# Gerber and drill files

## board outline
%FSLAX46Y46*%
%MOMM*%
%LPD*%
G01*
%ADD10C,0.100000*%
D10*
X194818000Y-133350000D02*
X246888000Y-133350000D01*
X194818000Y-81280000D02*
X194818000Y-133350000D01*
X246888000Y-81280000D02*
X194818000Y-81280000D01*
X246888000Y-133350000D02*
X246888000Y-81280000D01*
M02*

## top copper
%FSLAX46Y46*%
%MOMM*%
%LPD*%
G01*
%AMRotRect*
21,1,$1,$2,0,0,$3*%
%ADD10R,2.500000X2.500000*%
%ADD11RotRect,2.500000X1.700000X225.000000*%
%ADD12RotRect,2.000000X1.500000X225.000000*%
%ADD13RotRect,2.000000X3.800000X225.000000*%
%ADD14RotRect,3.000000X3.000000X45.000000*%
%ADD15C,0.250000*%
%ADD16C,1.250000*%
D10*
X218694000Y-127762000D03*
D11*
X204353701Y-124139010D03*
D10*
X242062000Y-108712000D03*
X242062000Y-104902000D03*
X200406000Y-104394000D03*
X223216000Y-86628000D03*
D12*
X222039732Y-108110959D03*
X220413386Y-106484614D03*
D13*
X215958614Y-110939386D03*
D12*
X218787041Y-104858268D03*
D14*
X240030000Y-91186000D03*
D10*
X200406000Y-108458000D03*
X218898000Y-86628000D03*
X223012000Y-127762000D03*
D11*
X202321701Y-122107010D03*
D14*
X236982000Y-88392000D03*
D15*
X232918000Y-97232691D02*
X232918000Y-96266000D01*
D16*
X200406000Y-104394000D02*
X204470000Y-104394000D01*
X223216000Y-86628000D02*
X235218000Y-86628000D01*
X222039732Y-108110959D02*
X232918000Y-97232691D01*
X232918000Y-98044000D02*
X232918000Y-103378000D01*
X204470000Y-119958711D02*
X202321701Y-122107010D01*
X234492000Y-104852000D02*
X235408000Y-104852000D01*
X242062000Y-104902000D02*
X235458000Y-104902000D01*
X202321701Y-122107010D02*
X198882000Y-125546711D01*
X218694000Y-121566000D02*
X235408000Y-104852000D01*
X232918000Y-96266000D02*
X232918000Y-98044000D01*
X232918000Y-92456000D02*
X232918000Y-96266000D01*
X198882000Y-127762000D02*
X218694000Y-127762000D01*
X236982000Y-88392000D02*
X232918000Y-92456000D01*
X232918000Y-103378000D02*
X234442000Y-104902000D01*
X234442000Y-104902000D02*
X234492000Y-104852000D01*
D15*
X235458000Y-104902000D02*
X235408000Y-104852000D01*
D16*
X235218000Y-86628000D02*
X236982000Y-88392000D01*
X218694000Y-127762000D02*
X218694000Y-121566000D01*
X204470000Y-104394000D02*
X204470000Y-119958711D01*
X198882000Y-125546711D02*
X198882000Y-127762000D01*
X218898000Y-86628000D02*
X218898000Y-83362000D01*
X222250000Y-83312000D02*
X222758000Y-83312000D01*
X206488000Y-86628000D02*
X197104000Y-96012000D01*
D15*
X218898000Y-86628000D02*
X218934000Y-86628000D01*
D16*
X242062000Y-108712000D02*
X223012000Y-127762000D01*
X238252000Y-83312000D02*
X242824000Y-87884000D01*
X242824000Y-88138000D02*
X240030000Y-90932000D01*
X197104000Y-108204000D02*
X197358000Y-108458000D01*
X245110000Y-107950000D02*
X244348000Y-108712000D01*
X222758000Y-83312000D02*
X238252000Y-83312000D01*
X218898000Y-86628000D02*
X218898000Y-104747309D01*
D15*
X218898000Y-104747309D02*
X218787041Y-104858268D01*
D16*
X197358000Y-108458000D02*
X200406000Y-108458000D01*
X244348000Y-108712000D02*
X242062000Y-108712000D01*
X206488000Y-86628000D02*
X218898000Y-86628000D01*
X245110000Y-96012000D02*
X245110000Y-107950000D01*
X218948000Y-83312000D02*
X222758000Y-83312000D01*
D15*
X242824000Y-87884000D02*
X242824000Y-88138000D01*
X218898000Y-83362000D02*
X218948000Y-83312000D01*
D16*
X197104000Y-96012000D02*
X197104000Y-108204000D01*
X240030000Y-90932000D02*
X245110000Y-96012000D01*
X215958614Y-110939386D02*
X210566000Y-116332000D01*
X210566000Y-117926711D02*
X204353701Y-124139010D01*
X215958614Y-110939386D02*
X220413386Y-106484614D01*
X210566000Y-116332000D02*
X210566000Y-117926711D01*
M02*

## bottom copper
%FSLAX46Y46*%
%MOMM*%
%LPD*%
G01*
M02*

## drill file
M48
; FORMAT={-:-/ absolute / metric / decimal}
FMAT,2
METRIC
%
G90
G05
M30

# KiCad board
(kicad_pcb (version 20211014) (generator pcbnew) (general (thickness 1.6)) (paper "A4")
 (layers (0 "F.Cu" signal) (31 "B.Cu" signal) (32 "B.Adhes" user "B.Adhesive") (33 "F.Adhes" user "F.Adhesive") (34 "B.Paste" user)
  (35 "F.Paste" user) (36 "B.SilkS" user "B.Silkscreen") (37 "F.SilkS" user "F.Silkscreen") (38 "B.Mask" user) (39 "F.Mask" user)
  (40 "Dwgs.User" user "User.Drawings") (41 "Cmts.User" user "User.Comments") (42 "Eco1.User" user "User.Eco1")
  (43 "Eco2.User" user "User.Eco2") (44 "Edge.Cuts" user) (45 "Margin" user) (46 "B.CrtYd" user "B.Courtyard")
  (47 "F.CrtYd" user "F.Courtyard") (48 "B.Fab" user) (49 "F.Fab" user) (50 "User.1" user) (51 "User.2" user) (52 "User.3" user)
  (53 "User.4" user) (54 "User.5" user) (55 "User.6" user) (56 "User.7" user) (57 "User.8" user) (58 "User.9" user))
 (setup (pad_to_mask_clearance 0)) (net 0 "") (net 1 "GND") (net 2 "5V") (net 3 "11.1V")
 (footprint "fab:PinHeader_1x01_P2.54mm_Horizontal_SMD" (layer "F.Cu") (at 218.694 127.762 -90)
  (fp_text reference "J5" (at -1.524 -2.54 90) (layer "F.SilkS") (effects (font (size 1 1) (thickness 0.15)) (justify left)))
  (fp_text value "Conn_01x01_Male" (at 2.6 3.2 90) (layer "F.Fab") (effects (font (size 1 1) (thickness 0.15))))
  (pad "1" smd rect locked (at 0 0 270) (size 2.5 2.5) (layers "F.Cu" "F.Paste" "F.Mask") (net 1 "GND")))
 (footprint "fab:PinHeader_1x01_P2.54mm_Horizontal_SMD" (layer "F.Cu") (at 204.353701 124.13901 -135)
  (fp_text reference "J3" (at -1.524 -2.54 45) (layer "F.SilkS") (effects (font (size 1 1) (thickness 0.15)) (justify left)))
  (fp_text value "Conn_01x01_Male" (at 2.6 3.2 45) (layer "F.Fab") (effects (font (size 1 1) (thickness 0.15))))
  (pad "1" smd rect locked (at 0 0 225) (size 2.5 1.7) (layers "F.Cu" "F.Paste" "F.Mask") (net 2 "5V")))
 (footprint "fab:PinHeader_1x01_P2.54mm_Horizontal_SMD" (layer "F.Cu") (at 242.062 108.712)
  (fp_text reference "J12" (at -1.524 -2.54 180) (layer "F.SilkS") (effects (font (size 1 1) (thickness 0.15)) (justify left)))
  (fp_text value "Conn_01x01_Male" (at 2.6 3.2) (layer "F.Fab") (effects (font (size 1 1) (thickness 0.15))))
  (pad "1" smd rect locked (at 0 0) (size 2.5 2.5) (layers "F.Cu" "F.Paste" "F.Mask") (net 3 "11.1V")))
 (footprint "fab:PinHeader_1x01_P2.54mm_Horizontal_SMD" (layer "F.Cu") (at 242.062 104.902)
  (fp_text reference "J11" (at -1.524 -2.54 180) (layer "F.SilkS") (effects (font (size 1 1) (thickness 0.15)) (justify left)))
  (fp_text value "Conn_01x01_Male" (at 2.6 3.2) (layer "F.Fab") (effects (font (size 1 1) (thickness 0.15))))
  (pad "1" smd rect locked (at 0 0) (size 2.5 2.5) (layers "F.Cu" "F.Paste" "F.Mask") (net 1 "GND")))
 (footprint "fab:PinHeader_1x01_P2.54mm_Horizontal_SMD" (layer "F.Cu") (at 200.406 104.394 180)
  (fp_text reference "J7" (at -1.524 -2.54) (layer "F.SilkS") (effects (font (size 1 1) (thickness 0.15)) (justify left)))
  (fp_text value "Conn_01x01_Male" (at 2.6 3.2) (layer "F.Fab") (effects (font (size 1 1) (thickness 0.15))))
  (pad "1" smd rect locked (at 0 0 180) (size 2.5 2.5) (layers "F.Cu" "F.Paste" "F.Mask") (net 1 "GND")))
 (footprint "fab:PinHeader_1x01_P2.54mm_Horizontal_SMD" (layer "F.Cu") (at 223.216 86.628 90)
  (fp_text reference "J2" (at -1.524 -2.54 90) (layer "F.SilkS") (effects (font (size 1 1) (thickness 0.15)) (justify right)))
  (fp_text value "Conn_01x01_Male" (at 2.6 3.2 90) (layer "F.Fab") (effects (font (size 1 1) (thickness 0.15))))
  (pad "1" smd rect locked (at 0 0 90) (size 2.5 2.5) (layers "F.Cu" "F.Paste" "F.Mask") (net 1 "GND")))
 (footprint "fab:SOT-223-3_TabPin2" (layer "F.Cu") (at 218.186 108.712 -135)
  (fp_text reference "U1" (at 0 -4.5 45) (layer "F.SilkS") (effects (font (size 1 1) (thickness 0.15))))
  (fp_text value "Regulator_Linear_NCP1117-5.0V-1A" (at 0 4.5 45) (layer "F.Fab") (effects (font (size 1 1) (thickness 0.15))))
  (pad "1" smd rect locked (at -3.15 -2.3 225) (size 2 1.5) (layers "F.Cu" "F.Paste" "F.Mask") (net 1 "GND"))
  (pad "2" smd rect locked (at -3.149999 0 225) (size 2 1.5) (layers "F.Cu" "F.Paste" "F.Mask") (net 2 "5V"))
  (pad "2" smd rect locked (at 3.149999 0 225) (size 2 3.8) (layers "F.Cu" "F.Paste" "F.Mask") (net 2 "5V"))
  (pad "3" smd rect locked (at -3.15 2.3 225) (size 2 1.5) (layers "F.Cu" "F.Paste" "F.Mask") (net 3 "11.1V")))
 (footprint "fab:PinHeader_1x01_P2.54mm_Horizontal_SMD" (layer "F.Cu") (at 240.03 91.186 45)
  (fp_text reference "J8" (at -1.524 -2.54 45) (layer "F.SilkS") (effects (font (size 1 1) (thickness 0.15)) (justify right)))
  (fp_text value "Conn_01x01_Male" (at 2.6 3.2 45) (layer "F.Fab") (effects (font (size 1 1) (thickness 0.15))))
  (pad "1" smd rect locked (at 0 0 45) (size 3 3) (layers "F.Cu" "F.Paste" "F.Mask") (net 3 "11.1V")))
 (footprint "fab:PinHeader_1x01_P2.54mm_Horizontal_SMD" (layer "F.Cu") (at 200.406 108.458 180)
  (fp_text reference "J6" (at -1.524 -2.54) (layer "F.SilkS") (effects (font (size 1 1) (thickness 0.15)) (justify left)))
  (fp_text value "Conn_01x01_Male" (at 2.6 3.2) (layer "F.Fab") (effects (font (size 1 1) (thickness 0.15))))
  (pad "1" smd rect locked (at 0 0 180) (size 2.5 2.5) (layers "F.Cu" "F.Paste" "F.Mask") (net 3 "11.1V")))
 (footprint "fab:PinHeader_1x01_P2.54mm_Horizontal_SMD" (layer "F.Cu") (at 218.898 86.628 90)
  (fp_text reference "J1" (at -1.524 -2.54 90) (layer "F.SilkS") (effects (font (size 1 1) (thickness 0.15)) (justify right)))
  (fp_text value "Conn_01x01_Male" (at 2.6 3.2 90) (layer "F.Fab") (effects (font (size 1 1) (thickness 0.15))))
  (pad "1" smd rect locked (at 0 0 90) (size 2.5 2.5) (layers "F.Cu" "F.Paste" "F.Mask") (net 3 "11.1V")))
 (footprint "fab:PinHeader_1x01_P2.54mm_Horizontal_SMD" (layer "F.Cu") (at 223.012 127.762 -90)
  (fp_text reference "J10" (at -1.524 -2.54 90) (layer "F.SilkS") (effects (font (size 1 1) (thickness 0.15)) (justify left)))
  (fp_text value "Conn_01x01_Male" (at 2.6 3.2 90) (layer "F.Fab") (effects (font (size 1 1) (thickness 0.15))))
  (pad "1" smd rect locked (at 0 0 270) (size 2.5 2.5) (layers "F.Cu" "F.Paste" "F.Mask") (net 3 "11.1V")))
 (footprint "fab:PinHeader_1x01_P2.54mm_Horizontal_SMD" (layer "F.Cu") (at 202.321701 122.10701 -135)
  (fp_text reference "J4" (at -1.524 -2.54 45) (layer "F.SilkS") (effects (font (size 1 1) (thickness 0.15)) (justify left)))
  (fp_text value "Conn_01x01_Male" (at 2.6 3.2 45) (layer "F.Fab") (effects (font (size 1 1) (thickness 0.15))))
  (pad "1" smd rect locked (at 0 0 225) (size 2.5 1.7) (layers "F.Cu" "F.Paste" "F.Mask") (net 1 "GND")))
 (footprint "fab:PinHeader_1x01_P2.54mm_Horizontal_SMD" (layer "F.Cu") (at 236.982 88.392 45)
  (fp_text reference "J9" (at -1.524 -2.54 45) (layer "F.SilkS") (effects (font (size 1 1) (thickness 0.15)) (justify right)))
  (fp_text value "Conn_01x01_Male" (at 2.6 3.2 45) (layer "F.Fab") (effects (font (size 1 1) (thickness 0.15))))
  (pad "1" smd rect locked (at 0 0 45) (size 3 3) (layers "F.Cu" "F.Paste" "F.Mask") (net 1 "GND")))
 (gr_line (start 194.818 133.35) (end 246.888 133.35) (layer "Edge.Cuts") (width 0.1))
 (gr_line (start 194.818 81.28) (end 194.818 133.35) (layer "Edge.Cuts") (width 0.1))
 (gr_line (start 246.888 81.28) (end 194.818 81.28) (layer "Edge.Cuts") (width 0.1))
 (gr_line (start 246.888 133.35) (end 246.888 81.28) (layer "Edge.Cuts") (width 0.1))
 (segment (start 232.918 97.232691) (end 232.918 96.266) (width 0.25) (layer "F.Cu") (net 1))
 (segment (start 200.406 104.394) (end 204.47 104.394) (width 1.25) (layer "F.Cu") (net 1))
 (segment (start 223.216 86.628) (end 235.218 86.628) (width 1.25) (layer "F.Cu") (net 1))
 (segment (start 222.039732 108.110959) (end 232.918 97.232691) (width 1.25) (layer "F.Cu") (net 1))
 (segment (start 232.918 98.044) (end 232.918 103.378) (width 1.25) (layer "F.Cu") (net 1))
 (segment (start 204.47 119.958711) (end 202.321701 122.10701) (width 1.25) (layer "F.Cu") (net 1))
 (segment (start 234.492 104.852) (end 235.408 104.852) (width 1.25) (layer "F.Cu") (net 1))
 (segment (start 242.062 104.902) (end 235.458 104.902) (width 1.25) (layer "F.Cu") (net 1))
 (segment (start 202.321701 122.10701) (end 198.882 125.546711) (width 1.25) (layer "F.Cu") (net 1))
 (segment (start 218.694 121.566) (end 235.408 104.852) (width 1.25) (layer "F.Cu") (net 1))
 (segment (start 232.918 96.266) (end 232.918 98.044) (width 1.25) (layer "F.Cu") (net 1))
 (segment (start 232.918 92.456) (end 232.918 96.266) (width 1.25) (layer "F.Cu") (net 1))
 (segment (start 198.882 127.762) (end 218.694 127.762) (width 1.25) (layer "F.Cu") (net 1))
 (segment (start 236.982 88.392) (end 232.918 92.456) (width 1.25) (layer "F.Cu") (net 1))
 (segment (start 232.918 103.378) (end 234.442 104.902) (width 1.25) (layer "F.Cu") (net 1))
 (segment (start 234.442 104.902) (end 234.492 104.852) (width 1.25) (layer "F.Cu") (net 1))
 (segment (start 235.458 104.902) (end 235.408 104.852) (width 0.25) (layer "F.Cu") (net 1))
 (segment (start 235.218 86.628) (end 236.982 88.392) (width 1.25) (layer "F.Cu") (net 1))
 (segment (start 218.694 127.762) (end 218.694 121.566) (width 1.25) (layer "F.Cu") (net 1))
 (segment (start 204.47 104.394) (end 204.47 119.958711) (width 1.25) (layer "F.Cu") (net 1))
 (segment (start 198.882 125.546711) (end 198.882 127.762) (width 1.25) (layer "F.Cu") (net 1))
 (segment (start 218.898 86.628) (end 218.898 83.362) (width 1.25) (layer "F.Cu") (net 3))
 (segment (start 222.25 83.312) (end 222.758 83.312) (width 1.25) (layer "F.Cu") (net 3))
 (segment (start 206.488 86.628) (end 197.104 96.012) (width 1.25) (layer "F.Cu") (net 3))
 (segment (start 218.898 86.628) (end 218.934 86.628) (width 0.25) (layer "F.Cu") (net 3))
 (segment (start 242.062 108.712) (end 223.012 127.762) (width 1.25) (layer "F.Cu") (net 3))
 (segment (start 238.252 83.312) (end 242.824 87.884) (width 1.25) (layer "F.Cu") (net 3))
 (segment (start 242.824 88.138) (end 240.03 90.932) (width 1.25) (layer "F.Cu") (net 3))
 (segment (start 197.104 108.204) (end 197.358 108.458) (width 1.25) (layer "F.Cu") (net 3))
 (segment (start 245.11 107.95) (end 244.348 108.712) (width 1.25) (layer "F.Cu") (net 3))
 (segment (start 222.758 83.312) (end 238.252 83.312) (width 1.25) (layer "F.Cu") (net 3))
 (segment (start 218.898 86.628) (end 218.898 104.747309) (width 1.25) (layer "F.Cu") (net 3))
 (segment (start 218.898 104.747309) (end 218.787041 104.858268) (width 0.25) (layer "F.Cu") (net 3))
 (segment (start 197.358 108.458) (end 200.406 108.458) (width 1.25) (layer "F.Cu") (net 3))
 (segment (start 244.348 108.712) (end 242.062 108.712) (width 1.25) (layer "F.Cu") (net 3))
 (segment (start 206.488 86.628) (end 218.898 86.628) (width 1.25) (layer "F.Cu") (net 3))
 (segment (start 245.11 96.012) (end 245.11 107.95) (width 1.25) (layer "F.Cu") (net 3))
 (segment (start 218.948 83.312) (end 222.758 83.312) (width 1.25) (layer "F.Cu") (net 3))
 (segment (start 242.824 87.884) (end 242.824 88.138) (width 0.25) (layer "F.Cu") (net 3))
 (segment (start 218.898 83.362) (end 218.948 83.312) (width 0.25) (layer "F.Cu") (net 3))
 (segment (start 197.104 96.012) (end 197.104 108.204) (width 1.25) (layer "F.Cu") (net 3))
 (segment (start 240.03 90.932) (end 245.11 96.012) (width 1.25) (layer "F.Cu") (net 3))
 (segment (start 215.958614 110.939386) (end 210.566 116.332) (width 1.25) (layer "F.Cu") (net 2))
 (segment (start 210.566 117.926711) (end 204.353701 124.13901) (width 1.25) (layer "F.Cu") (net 2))
 (segment (start 215.958614 110.939386) (end 220.413386 106.484614) (width 1.25) (layer "F.Cu") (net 2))
 (segment (start 210.566 116.332) (end 210.566 117.926711) (width 1.25) (layer "F.Cu") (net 2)))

